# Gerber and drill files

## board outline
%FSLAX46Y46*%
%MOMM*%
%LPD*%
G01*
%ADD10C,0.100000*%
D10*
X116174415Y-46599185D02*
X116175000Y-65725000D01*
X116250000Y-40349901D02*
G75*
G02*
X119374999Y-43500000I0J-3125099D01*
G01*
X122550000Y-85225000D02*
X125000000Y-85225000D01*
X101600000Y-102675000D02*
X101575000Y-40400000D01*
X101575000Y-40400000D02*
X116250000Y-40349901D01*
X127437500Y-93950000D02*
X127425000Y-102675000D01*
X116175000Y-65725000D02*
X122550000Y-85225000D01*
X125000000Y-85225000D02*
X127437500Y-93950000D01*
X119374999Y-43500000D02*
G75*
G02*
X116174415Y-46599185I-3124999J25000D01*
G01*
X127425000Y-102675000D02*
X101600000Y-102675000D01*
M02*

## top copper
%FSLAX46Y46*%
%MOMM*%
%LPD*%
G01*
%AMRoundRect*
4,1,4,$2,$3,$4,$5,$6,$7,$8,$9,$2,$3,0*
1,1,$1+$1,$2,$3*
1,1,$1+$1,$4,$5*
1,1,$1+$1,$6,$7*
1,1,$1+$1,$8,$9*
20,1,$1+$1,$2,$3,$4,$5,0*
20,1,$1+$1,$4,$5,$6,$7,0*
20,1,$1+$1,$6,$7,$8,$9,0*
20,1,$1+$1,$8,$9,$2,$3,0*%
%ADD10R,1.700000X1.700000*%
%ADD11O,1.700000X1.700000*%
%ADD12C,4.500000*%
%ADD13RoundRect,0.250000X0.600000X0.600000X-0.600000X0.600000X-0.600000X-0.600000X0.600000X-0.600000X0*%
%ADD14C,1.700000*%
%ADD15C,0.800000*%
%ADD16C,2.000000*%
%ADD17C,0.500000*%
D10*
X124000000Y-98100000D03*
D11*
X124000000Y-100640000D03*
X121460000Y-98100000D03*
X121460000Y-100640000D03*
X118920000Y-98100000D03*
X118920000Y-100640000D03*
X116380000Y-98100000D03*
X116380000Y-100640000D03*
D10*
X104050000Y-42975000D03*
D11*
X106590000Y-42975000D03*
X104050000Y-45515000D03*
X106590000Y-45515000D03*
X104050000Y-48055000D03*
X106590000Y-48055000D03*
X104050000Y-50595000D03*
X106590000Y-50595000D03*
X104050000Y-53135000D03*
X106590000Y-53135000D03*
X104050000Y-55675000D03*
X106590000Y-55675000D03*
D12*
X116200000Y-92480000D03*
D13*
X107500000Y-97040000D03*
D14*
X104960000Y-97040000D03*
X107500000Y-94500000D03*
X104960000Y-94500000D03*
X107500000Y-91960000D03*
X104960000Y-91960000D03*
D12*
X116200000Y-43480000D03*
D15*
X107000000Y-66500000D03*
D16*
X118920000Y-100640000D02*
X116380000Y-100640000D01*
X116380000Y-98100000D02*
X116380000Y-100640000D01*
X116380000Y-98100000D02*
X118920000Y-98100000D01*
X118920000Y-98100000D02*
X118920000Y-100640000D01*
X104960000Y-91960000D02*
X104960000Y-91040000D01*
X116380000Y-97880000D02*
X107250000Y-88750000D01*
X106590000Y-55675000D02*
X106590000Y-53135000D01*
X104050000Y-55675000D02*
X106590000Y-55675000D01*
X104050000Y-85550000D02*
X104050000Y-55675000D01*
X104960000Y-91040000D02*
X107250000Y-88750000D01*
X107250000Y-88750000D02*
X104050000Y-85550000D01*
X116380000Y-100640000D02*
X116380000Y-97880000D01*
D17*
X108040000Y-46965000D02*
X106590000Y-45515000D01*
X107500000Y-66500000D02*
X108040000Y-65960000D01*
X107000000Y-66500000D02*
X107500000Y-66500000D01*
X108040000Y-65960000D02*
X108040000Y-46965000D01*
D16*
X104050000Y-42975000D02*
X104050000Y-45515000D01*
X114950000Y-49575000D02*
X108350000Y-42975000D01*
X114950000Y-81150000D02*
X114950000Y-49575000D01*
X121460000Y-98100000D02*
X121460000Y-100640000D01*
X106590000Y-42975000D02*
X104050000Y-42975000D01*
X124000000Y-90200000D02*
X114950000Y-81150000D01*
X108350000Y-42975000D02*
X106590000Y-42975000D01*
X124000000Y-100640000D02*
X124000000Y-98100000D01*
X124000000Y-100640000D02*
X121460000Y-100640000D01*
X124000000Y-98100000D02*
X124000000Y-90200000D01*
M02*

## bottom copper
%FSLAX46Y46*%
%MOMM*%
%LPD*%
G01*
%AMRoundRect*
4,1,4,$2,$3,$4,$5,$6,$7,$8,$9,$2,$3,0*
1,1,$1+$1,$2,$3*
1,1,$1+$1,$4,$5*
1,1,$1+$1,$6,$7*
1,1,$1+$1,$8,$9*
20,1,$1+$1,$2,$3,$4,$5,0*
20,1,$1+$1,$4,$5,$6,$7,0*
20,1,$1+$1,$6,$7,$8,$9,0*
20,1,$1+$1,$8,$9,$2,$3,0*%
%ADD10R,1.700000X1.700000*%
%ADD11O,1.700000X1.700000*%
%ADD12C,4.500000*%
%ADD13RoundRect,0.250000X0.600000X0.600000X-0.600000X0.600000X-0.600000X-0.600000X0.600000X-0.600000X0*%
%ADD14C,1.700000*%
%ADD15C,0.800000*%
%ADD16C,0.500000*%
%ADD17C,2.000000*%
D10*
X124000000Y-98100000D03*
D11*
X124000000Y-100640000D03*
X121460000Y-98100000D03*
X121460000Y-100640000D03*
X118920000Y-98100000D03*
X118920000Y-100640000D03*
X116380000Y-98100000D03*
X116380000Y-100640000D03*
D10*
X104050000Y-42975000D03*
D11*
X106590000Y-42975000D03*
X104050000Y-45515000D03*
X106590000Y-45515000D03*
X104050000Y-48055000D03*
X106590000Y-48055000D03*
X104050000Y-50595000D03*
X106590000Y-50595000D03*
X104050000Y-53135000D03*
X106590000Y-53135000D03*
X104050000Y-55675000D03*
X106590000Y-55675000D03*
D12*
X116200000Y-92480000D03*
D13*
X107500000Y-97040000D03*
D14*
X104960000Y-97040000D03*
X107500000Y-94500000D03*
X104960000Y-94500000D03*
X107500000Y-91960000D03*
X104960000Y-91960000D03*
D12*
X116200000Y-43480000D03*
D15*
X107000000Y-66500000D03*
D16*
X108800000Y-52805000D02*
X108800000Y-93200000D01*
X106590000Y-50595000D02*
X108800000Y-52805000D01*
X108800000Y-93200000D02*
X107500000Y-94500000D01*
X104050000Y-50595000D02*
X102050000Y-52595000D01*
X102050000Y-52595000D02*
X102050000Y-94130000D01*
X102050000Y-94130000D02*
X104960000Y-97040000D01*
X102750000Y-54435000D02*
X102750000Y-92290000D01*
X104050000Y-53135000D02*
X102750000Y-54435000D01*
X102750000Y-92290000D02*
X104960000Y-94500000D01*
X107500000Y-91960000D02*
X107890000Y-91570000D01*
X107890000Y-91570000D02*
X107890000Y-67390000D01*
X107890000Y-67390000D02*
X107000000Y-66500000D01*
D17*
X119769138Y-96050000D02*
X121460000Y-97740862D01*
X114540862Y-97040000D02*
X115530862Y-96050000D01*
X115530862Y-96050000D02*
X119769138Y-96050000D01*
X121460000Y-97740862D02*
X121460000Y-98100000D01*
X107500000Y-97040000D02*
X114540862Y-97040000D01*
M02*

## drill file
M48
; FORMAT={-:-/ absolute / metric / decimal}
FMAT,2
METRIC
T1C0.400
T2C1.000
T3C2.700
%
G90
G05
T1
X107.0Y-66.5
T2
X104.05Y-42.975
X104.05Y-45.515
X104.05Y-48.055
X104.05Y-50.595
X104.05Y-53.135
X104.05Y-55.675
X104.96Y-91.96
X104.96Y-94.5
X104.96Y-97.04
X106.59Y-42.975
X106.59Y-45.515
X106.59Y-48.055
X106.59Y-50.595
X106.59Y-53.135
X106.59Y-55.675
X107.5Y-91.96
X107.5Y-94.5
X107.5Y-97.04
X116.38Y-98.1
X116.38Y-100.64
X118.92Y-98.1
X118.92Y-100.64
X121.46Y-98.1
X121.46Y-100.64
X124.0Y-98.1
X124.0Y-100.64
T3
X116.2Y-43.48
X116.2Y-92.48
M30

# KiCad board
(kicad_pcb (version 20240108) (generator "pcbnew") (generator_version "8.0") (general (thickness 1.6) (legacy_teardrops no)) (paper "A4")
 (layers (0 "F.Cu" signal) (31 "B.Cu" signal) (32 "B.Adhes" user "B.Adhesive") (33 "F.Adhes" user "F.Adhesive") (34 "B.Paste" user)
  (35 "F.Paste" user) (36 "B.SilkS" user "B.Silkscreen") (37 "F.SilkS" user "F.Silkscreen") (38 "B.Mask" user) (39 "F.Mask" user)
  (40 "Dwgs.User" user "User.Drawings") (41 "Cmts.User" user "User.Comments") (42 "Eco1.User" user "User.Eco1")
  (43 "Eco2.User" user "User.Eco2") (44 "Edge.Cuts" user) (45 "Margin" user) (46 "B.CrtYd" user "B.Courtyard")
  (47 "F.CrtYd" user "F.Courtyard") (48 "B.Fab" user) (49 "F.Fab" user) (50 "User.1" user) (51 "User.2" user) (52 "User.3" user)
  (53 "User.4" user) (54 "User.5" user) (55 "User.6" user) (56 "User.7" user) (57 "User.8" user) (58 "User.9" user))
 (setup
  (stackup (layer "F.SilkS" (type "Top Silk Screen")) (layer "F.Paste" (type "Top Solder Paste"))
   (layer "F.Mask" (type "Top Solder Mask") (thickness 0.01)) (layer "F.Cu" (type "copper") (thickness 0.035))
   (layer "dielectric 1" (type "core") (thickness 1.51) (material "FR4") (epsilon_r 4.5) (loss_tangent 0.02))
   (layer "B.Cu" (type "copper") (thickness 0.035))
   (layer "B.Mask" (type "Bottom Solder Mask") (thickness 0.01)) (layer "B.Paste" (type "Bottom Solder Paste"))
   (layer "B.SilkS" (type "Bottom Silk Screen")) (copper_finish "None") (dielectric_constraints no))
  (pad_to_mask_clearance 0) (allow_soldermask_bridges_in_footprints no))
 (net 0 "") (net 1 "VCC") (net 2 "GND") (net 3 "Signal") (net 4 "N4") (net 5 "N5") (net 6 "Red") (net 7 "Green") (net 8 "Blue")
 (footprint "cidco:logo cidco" (layer "F.Cu") (at 110.5 76.5)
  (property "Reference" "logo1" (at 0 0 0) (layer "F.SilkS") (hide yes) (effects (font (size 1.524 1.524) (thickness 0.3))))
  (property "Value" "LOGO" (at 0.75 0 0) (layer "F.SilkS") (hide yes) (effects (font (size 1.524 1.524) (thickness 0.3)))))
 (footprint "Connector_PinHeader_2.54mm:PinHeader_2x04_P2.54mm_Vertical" (layer "F.Cu") (at 124 98.1 -90)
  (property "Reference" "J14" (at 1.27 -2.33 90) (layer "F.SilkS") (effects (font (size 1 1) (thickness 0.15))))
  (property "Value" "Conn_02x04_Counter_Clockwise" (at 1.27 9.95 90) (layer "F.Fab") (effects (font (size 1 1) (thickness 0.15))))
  (pad "1" thru_hole rect (at 0 0 270) (size 1.7 1.7) (drill 1) (layers "*.Cu" "*.Mask") (remove_unused_layers no) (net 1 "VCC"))
  (pad "2" thru_hole oval (at 2.54 0 270) (size 1.7 1.7) (drill 1) (layers "*.Cu" "*.Mask") (remove_unused_layers no) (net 1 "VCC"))
  (pad "3" thru_hole oval (at 0 2.54 270) (size 1.7 1.7) (drill 1) (layers "*.Cu" "*.Mask") (remove_unused_layers no) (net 1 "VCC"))
  (pad "4" thru_hole oval (at 2.54 2.54 270) (size 1.7 1.7) (drill 1) (layers "*.Cu" "*.Mask") (remove_unused_layers no) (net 1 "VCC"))
  (pad "5" thru_hole oval (at 0 5.08 270) (size 1.7 1.7) (drill 1) (layers "*.Cu" "*.Mask") (remove_unused_layers no) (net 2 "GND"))
  (pad "6" thru_hole oval (at 2.54 5.08 270) (size 1.7 1.7) (drill 1) (layers "*.Cu" "*.Mask") (remove_unused_layers no) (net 2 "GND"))
  (pad "7" thru_hole oval (at 0 7.62 270) (size 1.7 1.7) (drill 1) (layers "*.Cu" "*.Mask") (remove_unused_layers no) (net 2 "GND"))
  (pad "8" thru_hole oval (at 2.54 7.62 270) (size 1.7 1.7) (drill 1) (layers "*.Cu" "*.Mask") (remove_unused_layers no) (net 2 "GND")))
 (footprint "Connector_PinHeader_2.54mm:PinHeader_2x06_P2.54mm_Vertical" (layer "F.Cu") (at 104.05 42.975)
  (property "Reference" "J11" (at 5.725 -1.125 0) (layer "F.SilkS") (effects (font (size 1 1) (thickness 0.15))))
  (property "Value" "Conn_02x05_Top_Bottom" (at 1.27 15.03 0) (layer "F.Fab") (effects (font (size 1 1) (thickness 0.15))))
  (pad "1" thru_hole rect (at 0 0) (size 1.7 1.7) (drill 1) (layers "*.Cu" "*.Mask") (remove_unused_layers no) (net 1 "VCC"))
  (pad "2" thru_hole oval (at 2.54 0) (size 1.7 1.7) (drill 1) (layers "*.Cu" "*.Mask") (remove_unused_layers no) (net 1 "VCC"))
  (pad "3" thru_hole oval (at 0 2.54) (size 1.7 1.7) (drill 1) (layers "*.Cu" "*.Mask") (remove_unused_layers no) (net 1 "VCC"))
  (pad "4" thru_hole oval (at 2.54 2.54) (size 1.7 1.7) (drill 1) (layers "*.Cu" "*.Mask") (remove_unused_layers no) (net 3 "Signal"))
  (pad "5" thru_hole oval (at 0 5.08) (size 1.7 1.7) (drill 1) (layers "*.Cu" "*.Mask") (remove_unused_layers no) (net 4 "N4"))
  (pad "6" thru_hole oval (at 2.54 5.08) (size 1.7 1.7) (drill 1) (layers "*.Cu" "*.Mask") (remove_unused_layers no) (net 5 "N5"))
  (pad "7" thru_hole oval (at 0 7.62) (size 1.7 1.7) (drill 1) (layers "*.Cu" "*.Mask") (remove_unused_layers no) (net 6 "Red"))
  (pad "8" thru_hole oval (at 2.54 7.62) (size 1.7 1.7) (drill 1) (layers "*.Cu" "*.Mask") (remove_unused_layers no) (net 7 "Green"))
  (pad "9" thru_hole oval (at 0 10.16) (size 1.7 1.7) (drill 1) (layers "*.Cu" "*.Mask") (remove_unused_layers no) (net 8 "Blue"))
  (pad "10" thru_hole oval (at 2.54 10.16) (size 1.7 1.7) (drill 1) (layers "*.Cu" "*.Mask") (remove_unused_layers no) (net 2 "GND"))
  (pad "11" thru_hole oval (at 0 12.7) (size 1.7 1.7) (drill 1) (layers "*.Cu" "*.Mask") (remove_unused_layers no) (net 2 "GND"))
  (pad "12" thru_hole oval (at 2.54 12.7) (size 1.7 1.7) (drill 1) (layers "*.Cu" "*.Mask") (remove_unused_layers no) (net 2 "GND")))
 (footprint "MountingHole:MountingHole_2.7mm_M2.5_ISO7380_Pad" (layer "F.Cu") (at 116.2 92.48)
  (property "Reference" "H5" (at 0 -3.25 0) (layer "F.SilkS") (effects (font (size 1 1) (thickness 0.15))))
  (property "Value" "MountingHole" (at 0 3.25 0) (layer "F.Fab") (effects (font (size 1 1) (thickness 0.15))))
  (pad "1" thru_hole circle (at 0 0) (size 4.5 4.5) (drill 2.7) (layers "*.Cu" "*.Mask") (remove_unused_layers no)))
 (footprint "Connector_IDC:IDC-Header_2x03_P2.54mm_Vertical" (layer "F.Cu") (at 107.5 97.04 180)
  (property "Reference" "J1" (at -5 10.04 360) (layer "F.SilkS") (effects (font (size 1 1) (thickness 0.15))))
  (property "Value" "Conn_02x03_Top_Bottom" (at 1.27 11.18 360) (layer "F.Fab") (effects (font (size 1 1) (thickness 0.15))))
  (pad "1" thru_hole roundrect (at 0 0 180) (size 1.7 1.7) (drill 1) (layers "*.Cu" "*.Mask") (remove_unused_layers no)
   (roundrect_rratio 0.147059) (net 1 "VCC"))
  (pad "2" thru_hole circle (at 2.54 0 180) (size 1.7 1.7) (drill 1) (layers "*.Cu" "*.Mask") (remove_unused_layers no) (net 6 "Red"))
  (pad "3" thru_hole circle (at 0 2.54 180) (size 1.7 1.7) (drill 1) (layers "*.Cu" "*.Mask") (remove_unused_layers no) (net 7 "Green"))
  (pad "4" thru_hole circle (at 2.54 2.54 180) (size 1.7 1.7) (drill 1) (layers "*.Cu" "*.Mask") (remove_unused_layers no) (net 8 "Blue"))
  (pad "5" thru_hole circle (at 0 5.08 180) (size 1.7 1.7) (drill 1) (layers "*.Cu" "*.Mask") (remove_unused_layers no) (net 3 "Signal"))
  (pad "6" thru_hole circle (at 2.54 5.08 180) (size 1.7 1.7) (drill 1) (layers "*.Cu" "*.Mask") (remove_unused_layers no) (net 2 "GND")))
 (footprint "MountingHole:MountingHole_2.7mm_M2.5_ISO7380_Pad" (layer "F.Cu") (at 116.2 43.48)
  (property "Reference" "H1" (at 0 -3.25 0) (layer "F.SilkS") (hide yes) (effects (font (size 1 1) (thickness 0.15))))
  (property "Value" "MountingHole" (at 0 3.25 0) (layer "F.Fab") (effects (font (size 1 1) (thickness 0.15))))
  (pad "1" thru_hole circle (at 0 0) (size 4.5 4.5) (drill 2.7) (layers "*.Cu" "*.Mask") (remove_unused_layers no)))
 (gr_line (start 116.174415 46.599185) (end 116.175 65.725) (stroke (width 0.1) (type default)) (layer "Edge.Cuts"))
 (gr_arc (start 116.25 40.349901) (mid 118.4686 41.274078) (end 119.374999 43.5) (stroke (width 0.1) (type default)) (layer "Edge.Cuts"))
 (gr_line (start 122.55 85.225) (end 125 85.225) (stroke (width 0.1) (type default)) (layer "Edge.Cuts"))
 (gr_line (start 101.6 102.675) (end 101.575 40.4) (stroke (width 0.1) (type default)) (layer "Edge.Cuts"))
 (gr_line (start 101.575 40.4) (end 116.25 40.349901) (stroke (width 0.1) (type default)) (layer "Edge.Cuts"))
 (gr_line (start 127.4375 93.95) (end 127.425 102.675) (stroke (width 0.1) (type default)) (layer "Edge.Cuts"))
 (gr_line (start 116.175 65.725) (end 122.55 85.225) (stroke (width 0.1) (type default)) (layer "Edge.Cuts"))
 (gr_line (start 125 85.225) (end 127.4375 93.95) (stroke (width 0.1) (type default)) (layer "Edge.Cuts"))
 (gr_arc (start 119.374999 43.5) (mid 118.423929 45.720056) (end 116.174415 46.599185) (stroke (width 0.1) (type default))
  (layer "Edge.Cuts"))
 (gr_line (start 127.425 102.675) (end 101.6 102.675) (stroke (width 0.1) (type default)) (layer "Edge.Cuts"))
 (segment (start 118.92 100.64) (end 116.38 100.64) (width 2) (layer "F.Cu") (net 2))
 (segment (start 116.38 98.1) (end 116.38 100.64) (width 2) (layer "F.Cu") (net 2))
 (segment (start 116.38 98.1) (end 118.92 98.1) (width 2) (layer "F.Cu") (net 2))
 (segment (start 118.92 98.1) (end 118.92 100.64) (width 2) (layer "F.Cu") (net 2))
 (segment (start 104.96 91.96) (end 104.96 91.04) (width 2) (layer "F.Cu") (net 2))
 (segment (start 116.38 97.88) (end 107.25 88.75) (width 2) (layer "F.Cu") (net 2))
 (segment (start 106.59 55.675) (end 106.59 53.135) (width 2) (layer "F.Cu") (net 2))
 (segment (start 104.05 55.675) (end 106.59 55.675) (width 2) (layer "F.Cu") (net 2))
 (segment (start 104.05 85.55) (end 104.05 55.675) (width 2) (layer "F.Cu") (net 2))
 (segment (start 104.96 91.04) (end 107.25 88.75) (width 2) (layer "F.Cu") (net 2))
 (segment (start 107.25 88.75) (end 104.05 85.55) (width 2) (layer "F.Cu") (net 2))
 (segment (start 116.38 100.64) (end 116.38 97.88) (width 2) (layer "F.Cu") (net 2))
 (segment (start 108.8 52.805) (end 108.8 93.2) (width 0.5) (layer "B.Cu") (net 7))
 (segment (start 106.59 50.595) (end 108.8 52.805) (width 0.5) (layer "B.Cu") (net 7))
 (segment (start 108.8 93.2) (end 107.5 94.5) (width 0.5) (layer "B.Cu") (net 7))
 (segment (start 104.05 50.595) (end 102.05 52.595) (width 0.5) (layer "B.Cu") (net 6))
 (segment (start 102.05 52.595) (end 102.05 94.13) (width 0.5) (layer "B.Cu") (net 6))
 (segment (start 102.05 94.13) (end 104.96 97.04) (width 0.5) (layer "B.Cu") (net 6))
 (segment (start 102.75 54.435) (end 102.75 92.29) (width 0.5) (layer "B.Cu") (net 8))
 (segment (start 104.05 53.135) (end 102.75 54.435) (width 0.5) (layer "B.Cu") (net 8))
 (segment (start 102.75 92.29) (end 104.96 94.5) (width 0.5) (layer "B.Cu") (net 8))
 (segment (start 108.04 46.965) (end 106.59 45.515) (width 0.5) (layer "F.Cu") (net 3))
 (segment (start 107.5 66.5) (end 108.04 65.96) (width 0.5) (layer "F.Cu") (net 3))
 (segment (start 107 66.5) (end 107.5 66.5) (width 0.5) (layer "F.Cu") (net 3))
 (segment (start 108.04 65.96) (end 108.04 46.965) (width 0.5) (layer "F.Cu") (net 3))
 (via (at 107 66.5) (size 0.8) (drill 0.4) (layers "F.Cu" "B.Cu") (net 3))
 (segment (start 107.5 91.96) (end 107.89 91.57) (width 0.5) (layer "B.Cu") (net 3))
 (segment (start 107.89 91.57) (end 107.89 67.39) (width 0.5) (layer "B.Cu") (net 3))
 (segment (start 107.89 67.39) (end 107 66.5) (width 0.5) (layer "B.Cu") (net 3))
 (segment (start 104.05 42.975) (end 104.05 45.515) (width 2) (layer "F.Cu") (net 1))
 (segment (start 114.95 49.575) (end 108.35 42.975) (width 2) (layer "F.Cu") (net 1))
 (segment (start 114.95 81.15) (end 114.95 49.575) (width 2) (layer "F.Cu") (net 1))
 (segment (start 121.46 98.1) (end 121.46 100.64) (width 2) (layer "F.Cu") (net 1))
 (segment (start 106.59 42.975) (end 104.05 42.975) (width 2) (layer "F.Cu") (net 1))
 (segment (start 124 90.2) (end 114.95 81.15) (width 2) (layer "F.Cu") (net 1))
 (segment (start 108.35 42.975) (end 106.59 42.975) (width 2) (layer "F.Cu") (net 1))
 (segment (start 124 100.64) (end 124 98.1) (width 2) (layer "F.Cu") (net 1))
 (segment (start 124 100.64) (end 121.46 100.64) (width 2) (layer "F.Cu") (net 1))
 (segment (start 124 98.1) (end 124 90.2) (width 2) (layer "F.Cu") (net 1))
 (segment (start 119.769138 96.05) (end 121.46 97.740862) (width 2) (layer "B.Cu") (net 1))
 (segment (start 114.540862 97.04) (end 115.530862 96.05) (width 2) (layer "B.Cu") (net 1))
 (segment (start 115.530862 96.05) (end 119.769138 96.05) (width 2) (layer "B.Cu") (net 1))
 (segment (start 121.46 97.740862) (end 121.46 98.1) (width 2) (layer "B.Cu") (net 1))
 (segment (start 107.5 97.04) (end 114.540862 97.04) (width 2) (layer "B.Cu") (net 1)))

